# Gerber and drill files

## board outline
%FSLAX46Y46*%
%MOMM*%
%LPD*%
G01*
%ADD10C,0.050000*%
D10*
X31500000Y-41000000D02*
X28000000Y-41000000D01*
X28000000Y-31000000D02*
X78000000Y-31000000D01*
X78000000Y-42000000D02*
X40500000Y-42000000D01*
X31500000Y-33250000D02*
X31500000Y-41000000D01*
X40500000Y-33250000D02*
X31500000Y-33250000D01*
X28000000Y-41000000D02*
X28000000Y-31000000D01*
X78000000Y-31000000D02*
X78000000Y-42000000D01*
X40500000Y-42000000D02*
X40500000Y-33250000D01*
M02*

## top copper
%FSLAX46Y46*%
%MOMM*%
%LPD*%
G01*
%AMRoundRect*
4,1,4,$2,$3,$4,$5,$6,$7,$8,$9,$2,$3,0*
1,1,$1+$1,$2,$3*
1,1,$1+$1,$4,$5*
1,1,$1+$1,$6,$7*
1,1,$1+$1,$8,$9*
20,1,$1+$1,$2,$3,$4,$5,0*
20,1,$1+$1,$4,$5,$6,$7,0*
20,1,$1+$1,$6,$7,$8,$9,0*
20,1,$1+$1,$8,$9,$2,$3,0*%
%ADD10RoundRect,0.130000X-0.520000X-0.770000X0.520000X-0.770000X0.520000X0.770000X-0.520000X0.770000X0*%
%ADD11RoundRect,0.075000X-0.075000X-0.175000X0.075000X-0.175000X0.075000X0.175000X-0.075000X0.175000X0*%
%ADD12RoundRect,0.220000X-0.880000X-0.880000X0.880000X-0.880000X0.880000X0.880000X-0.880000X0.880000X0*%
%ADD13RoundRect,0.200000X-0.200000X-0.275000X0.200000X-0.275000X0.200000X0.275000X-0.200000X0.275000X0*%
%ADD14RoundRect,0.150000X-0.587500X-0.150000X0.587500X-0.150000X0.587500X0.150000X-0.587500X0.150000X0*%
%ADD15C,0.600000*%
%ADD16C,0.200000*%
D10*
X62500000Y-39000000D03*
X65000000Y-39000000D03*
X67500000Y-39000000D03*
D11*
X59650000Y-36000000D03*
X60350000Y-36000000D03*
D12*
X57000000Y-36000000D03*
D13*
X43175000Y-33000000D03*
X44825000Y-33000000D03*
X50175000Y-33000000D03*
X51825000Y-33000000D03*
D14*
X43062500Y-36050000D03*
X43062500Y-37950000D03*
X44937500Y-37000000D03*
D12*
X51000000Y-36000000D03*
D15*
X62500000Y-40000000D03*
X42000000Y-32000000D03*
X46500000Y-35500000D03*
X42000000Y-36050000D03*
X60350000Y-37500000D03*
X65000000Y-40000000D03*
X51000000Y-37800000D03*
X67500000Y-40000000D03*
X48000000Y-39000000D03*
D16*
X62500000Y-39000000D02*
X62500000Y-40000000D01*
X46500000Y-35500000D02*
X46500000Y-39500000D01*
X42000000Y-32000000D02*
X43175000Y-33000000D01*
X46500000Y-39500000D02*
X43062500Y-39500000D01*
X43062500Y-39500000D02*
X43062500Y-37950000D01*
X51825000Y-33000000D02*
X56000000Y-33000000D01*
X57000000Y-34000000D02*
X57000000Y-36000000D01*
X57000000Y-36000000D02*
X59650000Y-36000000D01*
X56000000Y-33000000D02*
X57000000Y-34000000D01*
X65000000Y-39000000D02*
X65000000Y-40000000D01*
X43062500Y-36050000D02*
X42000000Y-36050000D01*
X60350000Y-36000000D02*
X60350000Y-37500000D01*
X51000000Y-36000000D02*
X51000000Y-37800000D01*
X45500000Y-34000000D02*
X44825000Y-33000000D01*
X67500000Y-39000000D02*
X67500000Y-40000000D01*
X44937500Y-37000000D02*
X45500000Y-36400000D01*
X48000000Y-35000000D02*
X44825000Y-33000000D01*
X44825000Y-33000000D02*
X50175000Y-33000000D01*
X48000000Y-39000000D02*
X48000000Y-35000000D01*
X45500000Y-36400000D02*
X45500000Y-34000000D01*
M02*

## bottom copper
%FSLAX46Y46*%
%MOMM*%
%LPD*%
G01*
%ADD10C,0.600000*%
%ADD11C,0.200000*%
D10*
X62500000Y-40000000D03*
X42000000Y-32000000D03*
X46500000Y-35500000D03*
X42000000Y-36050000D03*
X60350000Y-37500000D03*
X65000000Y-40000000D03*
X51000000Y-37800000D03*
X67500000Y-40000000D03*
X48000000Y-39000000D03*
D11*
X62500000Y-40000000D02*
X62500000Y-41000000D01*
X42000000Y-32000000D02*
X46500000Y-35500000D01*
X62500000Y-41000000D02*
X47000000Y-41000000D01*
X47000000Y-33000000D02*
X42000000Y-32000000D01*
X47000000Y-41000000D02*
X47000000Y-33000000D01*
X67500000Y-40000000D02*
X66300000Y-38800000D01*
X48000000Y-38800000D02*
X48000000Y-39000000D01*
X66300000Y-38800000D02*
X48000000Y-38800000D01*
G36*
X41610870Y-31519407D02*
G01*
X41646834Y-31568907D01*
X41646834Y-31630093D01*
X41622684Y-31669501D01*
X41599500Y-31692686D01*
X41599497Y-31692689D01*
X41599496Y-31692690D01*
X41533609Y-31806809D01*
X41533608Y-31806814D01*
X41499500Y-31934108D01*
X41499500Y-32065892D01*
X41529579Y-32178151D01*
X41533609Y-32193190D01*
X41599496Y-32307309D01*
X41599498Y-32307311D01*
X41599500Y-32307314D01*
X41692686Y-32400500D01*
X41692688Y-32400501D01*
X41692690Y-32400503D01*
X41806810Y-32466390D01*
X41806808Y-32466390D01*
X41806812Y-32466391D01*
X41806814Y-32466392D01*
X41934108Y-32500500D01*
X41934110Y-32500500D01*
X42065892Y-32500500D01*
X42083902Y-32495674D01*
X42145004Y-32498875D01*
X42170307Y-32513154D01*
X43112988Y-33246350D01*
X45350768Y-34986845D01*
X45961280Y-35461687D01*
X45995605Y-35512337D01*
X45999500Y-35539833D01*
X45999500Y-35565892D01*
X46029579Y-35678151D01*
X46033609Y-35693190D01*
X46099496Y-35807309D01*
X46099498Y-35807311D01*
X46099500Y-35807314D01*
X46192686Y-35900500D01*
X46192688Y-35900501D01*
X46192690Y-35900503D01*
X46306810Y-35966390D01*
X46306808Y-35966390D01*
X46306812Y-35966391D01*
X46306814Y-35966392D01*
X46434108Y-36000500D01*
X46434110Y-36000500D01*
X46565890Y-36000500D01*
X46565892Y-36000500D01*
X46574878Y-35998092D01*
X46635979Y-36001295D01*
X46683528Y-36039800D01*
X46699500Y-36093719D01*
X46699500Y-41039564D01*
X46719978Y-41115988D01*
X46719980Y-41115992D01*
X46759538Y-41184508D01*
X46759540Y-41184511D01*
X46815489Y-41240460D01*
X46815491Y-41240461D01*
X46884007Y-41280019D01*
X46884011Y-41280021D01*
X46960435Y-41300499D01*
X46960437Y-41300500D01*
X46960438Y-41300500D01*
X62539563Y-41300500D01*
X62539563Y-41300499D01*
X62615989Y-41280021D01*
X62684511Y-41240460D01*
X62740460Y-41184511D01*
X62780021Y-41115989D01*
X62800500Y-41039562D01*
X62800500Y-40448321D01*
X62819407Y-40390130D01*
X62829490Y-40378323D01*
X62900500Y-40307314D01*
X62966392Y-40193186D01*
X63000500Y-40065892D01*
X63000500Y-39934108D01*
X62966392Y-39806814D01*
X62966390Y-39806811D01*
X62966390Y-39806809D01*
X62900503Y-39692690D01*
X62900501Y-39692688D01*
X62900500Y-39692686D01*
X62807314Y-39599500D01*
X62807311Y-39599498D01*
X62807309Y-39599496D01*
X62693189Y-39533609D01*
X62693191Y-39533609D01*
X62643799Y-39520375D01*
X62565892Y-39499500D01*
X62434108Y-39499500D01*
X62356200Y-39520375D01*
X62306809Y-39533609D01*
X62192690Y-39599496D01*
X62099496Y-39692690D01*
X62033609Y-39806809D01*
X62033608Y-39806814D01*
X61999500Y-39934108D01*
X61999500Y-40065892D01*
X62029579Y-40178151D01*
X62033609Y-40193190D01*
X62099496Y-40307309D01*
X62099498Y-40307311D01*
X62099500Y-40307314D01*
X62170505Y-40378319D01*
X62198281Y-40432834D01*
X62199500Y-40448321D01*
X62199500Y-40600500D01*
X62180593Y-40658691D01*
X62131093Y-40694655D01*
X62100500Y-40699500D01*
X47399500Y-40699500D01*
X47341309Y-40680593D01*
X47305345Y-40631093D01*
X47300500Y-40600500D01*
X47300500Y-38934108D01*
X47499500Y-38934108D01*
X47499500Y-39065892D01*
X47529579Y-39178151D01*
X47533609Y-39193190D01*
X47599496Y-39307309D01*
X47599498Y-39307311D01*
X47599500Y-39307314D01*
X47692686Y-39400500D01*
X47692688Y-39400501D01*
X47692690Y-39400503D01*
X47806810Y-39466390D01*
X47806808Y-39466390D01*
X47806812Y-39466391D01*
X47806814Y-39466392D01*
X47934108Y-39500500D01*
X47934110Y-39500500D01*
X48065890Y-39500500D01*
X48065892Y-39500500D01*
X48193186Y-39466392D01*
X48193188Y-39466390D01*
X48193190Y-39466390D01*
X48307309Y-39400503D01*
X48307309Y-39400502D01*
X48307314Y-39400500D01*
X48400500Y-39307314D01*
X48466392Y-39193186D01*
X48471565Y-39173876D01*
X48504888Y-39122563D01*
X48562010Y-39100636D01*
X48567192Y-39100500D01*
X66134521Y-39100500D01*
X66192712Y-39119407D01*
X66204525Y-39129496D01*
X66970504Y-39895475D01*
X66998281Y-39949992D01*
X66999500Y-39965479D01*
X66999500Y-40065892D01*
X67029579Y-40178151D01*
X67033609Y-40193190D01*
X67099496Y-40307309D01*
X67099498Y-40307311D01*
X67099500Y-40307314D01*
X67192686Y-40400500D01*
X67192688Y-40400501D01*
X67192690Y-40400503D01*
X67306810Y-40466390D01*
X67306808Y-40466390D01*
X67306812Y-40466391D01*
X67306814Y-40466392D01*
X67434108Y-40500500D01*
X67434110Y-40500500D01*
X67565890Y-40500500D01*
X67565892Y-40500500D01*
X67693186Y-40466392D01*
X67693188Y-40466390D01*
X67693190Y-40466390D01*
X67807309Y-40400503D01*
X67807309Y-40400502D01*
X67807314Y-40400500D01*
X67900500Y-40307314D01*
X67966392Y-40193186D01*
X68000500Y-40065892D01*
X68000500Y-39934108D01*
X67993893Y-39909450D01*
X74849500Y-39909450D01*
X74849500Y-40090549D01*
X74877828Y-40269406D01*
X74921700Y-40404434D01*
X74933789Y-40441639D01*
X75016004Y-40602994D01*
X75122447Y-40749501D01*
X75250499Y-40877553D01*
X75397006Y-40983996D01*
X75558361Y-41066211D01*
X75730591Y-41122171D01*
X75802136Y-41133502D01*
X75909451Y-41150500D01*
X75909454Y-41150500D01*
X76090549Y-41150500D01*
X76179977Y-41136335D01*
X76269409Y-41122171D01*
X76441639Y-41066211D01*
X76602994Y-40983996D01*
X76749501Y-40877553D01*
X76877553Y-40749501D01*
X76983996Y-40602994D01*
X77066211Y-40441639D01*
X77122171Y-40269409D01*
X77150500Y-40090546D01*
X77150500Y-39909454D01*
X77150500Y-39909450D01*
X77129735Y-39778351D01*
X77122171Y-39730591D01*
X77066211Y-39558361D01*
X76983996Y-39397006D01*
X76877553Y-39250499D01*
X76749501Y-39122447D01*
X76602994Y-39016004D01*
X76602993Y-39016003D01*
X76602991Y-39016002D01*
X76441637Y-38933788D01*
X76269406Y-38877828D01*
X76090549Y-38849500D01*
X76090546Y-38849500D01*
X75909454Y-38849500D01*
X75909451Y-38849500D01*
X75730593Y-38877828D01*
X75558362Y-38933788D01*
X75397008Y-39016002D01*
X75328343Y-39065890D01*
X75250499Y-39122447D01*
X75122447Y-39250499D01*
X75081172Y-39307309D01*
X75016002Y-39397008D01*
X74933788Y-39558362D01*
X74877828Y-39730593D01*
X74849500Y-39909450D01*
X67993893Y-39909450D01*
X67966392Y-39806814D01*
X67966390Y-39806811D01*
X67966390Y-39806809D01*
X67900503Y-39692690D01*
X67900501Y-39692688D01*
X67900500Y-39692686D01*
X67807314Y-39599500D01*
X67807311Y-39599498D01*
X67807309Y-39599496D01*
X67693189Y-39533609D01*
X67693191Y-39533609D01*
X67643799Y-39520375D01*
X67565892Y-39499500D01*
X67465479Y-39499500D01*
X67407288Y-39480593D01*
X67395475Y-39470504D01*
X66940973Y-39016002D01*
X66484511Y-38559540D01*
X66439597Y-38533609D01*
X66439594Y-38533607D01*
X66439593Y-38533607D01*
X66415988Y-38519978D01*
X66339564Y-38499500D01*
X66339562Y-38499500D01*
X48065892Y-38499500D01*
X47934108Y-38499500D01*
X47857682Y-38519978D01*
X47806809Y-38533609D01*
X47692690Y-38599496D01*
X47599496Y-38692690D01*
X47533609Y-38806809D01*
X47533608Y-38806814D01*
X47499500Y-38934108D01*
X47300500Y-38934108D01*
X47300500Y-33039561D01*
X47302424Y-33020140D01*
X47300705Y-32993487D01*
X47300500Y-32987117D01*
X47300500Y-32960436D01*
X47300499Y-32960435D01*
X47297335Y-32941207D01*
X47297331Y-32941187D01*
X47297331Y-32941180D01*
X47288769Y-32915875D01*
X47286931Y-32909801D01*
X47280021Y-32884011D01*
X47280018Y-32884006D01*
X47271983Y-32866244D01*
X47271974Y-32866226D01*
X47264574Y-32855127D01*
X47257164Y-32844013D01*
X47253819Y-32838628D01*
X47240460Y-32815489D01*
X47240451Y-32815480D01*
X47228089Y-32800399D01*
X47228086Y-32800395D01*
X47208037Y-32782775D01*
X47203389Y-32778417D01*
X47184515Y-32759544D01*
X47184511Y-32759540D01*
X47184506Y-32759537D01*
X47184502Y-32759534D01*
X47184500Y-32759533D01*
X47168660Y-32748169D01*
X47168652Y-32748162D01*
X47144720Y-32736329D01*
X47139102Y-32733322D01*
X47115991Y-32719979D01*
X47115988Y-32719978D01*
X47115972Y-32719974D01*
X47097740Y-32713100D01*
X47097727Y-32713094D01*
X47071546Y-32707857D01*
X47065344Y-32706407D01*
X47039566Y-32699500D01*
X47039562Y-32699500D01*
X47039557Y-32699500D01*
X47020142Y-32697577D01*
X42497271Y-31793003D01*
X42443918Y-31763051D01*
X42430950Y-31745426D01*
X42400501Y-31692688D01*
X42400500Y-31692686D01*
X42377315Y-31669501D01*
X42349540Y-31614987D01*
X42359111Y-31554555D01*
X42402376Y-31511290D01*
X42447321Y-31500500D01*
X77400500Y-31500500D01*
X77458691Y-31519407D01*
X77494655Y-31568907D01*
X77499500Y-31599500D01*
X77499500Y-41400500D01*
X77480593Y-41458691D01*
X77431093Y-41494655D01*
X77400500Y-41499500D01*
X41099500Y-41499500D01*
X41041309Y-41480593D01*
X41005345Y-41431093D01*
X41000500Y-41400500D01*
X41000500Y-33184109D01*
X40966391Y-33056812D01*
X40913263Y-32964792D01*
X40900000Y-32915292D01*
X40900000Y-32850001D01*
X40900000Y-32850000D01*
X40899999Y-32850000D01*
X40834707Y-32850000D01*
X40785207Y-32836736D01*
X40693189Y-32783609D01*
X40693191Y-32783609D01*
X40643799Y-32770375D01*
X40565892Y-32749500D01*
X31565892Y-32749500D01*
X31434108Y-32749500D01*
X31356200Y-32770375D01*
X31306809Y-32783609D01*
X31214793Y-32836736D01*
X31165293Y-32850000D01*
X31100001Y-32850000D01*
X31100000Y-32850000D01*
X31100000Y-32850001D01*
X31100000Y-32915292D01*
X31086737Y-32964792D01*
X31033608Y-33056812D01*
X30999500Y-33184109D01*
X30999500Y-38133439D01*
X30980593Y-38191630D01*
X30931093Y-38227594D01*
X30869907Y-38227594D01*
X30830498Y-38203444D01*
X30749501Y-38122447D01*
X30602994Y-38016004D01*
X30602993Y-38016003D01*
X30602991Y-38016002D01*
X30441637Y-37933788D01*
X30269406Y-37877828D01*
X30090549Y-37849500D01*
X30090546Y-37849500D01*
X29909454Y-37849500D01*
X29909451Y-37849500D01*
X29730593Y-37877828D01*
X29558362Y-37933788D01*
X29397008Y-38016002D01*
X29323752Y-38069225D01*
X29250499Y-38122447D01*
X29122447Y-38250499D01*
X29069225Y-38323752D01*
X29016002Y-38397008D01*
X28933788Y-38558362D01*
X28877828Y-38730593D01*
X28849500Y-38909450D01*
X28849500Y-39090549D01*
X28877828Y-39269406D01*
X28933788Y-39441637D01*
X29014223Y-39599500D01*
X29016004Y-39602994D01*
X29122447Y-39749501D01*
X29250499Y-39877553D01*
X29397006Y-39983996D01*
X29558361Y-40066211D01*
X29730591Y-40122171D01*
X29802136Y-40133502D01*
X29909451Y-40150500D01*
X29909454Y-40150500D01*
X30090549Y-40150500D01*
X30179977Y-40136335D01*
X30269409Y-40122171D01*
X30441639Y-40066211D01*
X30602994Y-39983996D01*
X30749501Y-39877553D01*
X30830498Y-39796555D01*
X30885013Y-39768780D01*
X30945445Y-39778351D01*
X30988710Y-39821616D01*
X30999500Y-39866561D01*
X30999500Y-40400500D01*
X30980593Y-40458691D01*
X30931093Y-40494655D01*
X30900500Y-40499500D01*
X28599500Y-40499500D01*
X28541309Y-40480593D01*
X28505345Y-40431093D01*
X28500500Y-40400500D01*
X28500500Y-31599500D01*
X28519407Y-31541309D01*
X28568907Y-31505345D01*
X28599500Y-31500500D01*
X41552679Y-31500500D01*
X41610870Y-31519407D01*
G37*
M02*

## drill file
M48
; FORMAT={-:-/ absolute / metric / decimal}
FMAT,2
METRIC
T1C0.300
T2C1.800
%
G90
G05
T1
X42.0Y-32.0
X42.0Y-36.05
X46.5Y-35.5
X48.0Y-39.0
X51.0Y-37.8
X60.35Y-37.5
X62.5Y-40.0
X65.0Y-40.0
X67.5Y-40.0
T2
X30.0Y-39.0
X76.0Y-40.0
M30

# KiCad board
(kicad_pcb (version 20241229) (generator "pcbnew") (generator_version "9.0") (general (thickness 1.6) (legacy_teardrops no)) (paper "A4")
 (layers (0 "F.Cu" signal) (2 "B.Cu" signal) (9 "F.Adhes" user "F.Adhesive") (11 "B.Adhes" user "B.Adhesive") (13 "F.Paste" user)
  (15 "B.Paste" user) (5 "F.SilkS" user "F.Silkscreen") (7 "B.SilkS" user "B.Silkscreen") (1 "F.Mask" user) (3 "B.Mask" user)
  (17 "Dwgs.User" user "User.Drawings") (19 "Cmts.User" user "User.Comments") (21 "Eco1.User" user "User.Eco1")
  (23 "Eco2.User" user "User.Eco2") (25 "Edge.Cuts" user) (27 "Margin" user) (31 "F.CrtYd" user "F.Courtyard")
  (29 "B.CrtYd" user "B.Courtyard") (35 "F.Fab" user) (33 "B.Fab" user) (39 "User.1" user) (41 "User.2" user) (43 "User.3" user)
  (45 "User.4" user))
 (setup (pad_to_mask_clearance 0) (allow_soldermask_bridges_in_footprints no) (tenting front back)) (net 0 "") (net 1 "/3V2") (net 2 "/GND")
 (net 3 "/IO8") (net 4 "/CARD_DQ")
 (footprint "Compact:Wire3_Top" (layer "F.Cu") (at 65 39)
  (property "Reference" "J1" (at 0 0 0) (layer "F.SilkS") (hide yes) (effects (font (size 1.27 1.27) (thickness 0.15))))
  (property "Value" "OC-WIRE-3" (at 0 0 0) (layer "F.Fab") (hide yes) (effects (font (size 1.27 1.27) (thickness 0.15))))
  (pad "1" smd roundrect (at -2.5 0) (size 1.3 1.8) (layers "F.Cu" "F.Mask") (roundrect_rratio 0.1) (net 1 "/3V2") (thermal_bridge_angle 45))
  (pad "2" smd roundrect (at 0 0) (size 1.3 1.8) (layers "F.Cu" "F.Mask") (roundrect_rratio 0.1) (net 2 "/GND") (thermal_bridge_angle 45))
  (pad "3" smd roundrect (at 2.5 0) (size 1.3 1.8) (layers "F.Cu" "F.Mask") (roundrect_rratio 0.1) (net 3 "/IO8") (thermal_bridge_angle 45)))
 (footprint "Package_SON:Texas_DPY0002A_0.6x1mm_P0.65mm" (layer "F.Cu") (at 60 36)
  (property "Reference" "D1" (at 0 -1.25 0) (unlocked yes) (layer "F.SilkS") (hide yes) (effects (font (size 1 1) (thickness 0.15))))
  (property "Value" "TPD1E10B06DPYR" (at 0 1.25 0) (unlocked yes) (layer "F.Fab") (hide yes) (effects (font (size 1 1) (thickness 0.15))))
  (pad "1" smd roundrect (at -0.35 0) (size 0.3 0.5) (layers "F.Cu" "F.Mask" "F.Paste") (roundrect_rratio 0.25) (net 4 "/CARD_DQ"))
  (pad "2" smd roundrect (at 0.35 0) (size 0.3 0.5) (layers "F.Cu" "F.Mask" "F.Paste") (roundrect_rratio 0.25) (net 2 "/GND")))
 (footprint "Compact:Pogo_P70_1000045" (layer "F.Cu") (at 57 36)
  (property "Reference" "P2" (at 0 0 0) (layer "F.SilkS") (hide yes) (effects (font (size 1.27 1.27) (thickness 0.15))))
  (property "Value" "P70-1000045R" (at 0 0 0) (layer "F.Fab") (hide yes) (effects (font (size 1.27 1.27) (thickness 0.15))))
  (pad "1" smd roundrect (at 0 0) (size 2.2 2.2) (layers "F.Cu" "F.Mask" "F.Paste") (roundrect_rratio 0.1) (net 4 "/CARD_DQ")
   (thermal_bridge_angle 45)))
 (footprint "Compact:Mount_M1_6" (layer "F.Cu") (at 30 39)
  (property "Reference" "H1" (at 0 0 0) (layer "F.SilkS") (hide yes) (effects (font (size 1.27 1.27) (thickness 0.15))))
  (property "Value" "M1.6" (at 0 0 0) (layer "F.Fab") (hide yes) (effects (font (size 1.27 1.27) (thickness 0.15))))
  (pad "" np_thru_hole circle (at 0 0) (size 1.8 1.8) (drill 1.8) (layers "*.Cu")))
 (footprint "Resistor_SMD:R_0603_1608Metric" (layer "F.Cu") (at 44 33)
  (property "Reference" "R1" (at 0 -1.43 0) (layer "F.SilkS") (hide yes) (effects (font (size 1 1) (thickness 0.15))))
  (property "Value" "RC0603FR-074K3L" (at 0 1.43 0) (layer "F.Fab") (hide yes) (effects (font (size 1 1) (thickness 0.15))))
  (pad "1" smd roundrect (at -0.825 0) (size 0.8 0.95) (layers "F.Cu" "F.Mask" "F.Paste") (roundrect_rratio 0.25) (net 1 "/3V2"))
  (pad "2" smd roundrect (at 0.825 0) (size 0.8 0.95) (layers "F.Cu" "F.Mask" "F.Paste") (roundrect_rratio 0.25) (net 3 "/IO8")))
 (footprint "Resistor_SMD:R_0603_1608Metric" (layer "F.Cu") (at 51 33)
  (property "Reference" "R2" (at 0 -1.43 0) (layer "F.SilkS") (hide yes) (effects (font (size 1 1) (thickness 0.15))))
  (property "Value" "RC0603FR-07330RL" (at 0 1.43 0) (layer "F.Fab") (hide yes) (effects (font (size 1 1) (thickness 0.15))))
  (pad "1" smd roundrect (at -0.825 0) (size 0.8 0.95) (layers "F.Cu" "F.Mask" "F.Paste") (roundrect_rratio 0.25) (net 3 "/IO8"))
  (pad "2" smd roundrect (at 0.825 0) (size 0.8 0.95) (layers "F.Cu" "F.Mask" "F.Paste") (roundrect_rratio 0.25) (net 4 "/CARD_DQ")))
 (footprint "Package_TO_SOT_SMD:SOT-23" (layer "F.Cu") (at 44 37)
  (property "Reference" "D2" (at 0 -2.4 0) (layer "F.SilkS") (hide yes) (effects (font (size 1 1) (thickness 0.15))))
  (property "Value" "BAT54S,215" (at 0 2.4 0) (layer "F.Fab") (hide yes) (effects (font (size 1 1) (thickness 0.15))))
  (pad "1" smd roundrect (at -0.9375 -0.95) (size 1.475 0.6) (layers "F.Cu" "F.Mask" "F.Paste") (roundrect_rratio 0.25) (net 2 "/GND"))
  (pad "2" smd roundrect (at -0.9375 0.95) (size 1.475 0.6) (layers "F.Cu" "F.Mask" "F.Paste") (roundrect_rratio 0.25) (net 1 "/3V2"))
  (pad "3" smd roundrect (at 0.9375 0) (size 1.475 0.6) (layers "F.Cu" "F.Mask" "F.Paste") (roundrect_rratio 0.25) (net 3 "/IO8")))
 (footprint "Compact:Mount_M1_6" (layer "F.Cu") (at 76 40)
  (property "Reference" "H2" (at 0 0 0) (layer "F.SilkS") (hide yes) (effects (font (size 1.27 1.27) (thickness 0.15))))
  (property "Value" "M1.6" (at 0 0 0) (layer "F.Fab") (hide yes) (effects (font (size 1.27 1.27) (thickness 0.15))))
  (pad "" np_thru_hole circle (at 0 0) (size 1.8 1.8) (drill 1.8) (layers "*.Cu")))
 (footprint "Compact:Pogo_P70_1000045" (layer "F.Cu") (at 51 36)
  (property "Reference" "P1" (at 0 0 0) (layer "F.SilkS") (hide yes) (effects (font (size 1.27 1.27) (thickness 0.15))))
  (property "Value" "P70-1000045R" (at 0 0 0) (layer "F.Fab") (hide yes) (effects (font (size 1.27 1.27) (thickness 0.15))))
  (pad "1" smd roundrect (at 0 0) (size 2.2 2.2) (layers "F.Cu" "F.Mask" "F.Paste") (roundrect_rratio 0.1) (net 2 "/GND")
   (thermal_bridge_angle 45)))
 (gr_line (start 31.5 41) (end 28 41) (stroke (width 0.05) (type default)) (layer "Edge.Cuts"))
 (gr_line (start 28 31) (end 78 31) (stroke (width 0.05) (type default)) (layer "Edge.Cuts"))
 (gr_line (start 78 42) (end 40.5 42) (stroke (width 0.05) (type default)) (layer "Edge.Cuts"))
 (gr_line (start 31.5 33.25) (end 31.5 41) (stroke (width 0.05) (type default)) (layer "Edge.Cuts"))
 (gr_line (start 40.5 33.25) (end 31.5 33.25) (stroke (width 0.05) (type default)) (layer "Edge.Cuts"))
 (gr_line (start 28 41) (end 28 31) (stroke (width 0.05) (type default)) (layer "Edge.Cuts"))
 (gr_line (start 78 31) (end 78 42) (stroke (width 0.05) (type default)) (layer "Edge.Cuts"))
 (gr_line (start 40.5 42) (end 40.5 33.25) (stroke (width 0.05) (type default)) (layer "Edge.Cuts"))
 (segment (start 62.5 39) (end 62.5 40) (width 0.2) (layer "F.Cu") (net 1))
 (segment (start 46.5 35.5) (end 46.5 39.5) (width 0.2) (layer "F.Cu") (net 1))
 (segment (start 42 32) (end 43.175 33) (width 0.2) (layer "F.Cu") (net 1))
 (segment (start 46.5 39.5) (end 43.0625 39.5) (width 0.2) (layer "F.Cu") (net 1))
 (segment (start 43.0625 39.5) (end 43.0625 37.95) (width 0.2) (layer "F.Cu") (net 1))
 (via (at 62.5 40) (size 0.6) (drill 0.3) (layers "F.Cu" "B.Cu") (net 1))
 (via (at 42 32) (size 0.6) (drill 0.3) (layers "F.Cu" "B.Cu") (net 1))
 (via (at 46.5 35.5) (size 0.6) (drill 0.3) (layers "F.Cu" "B.Cu") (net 1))
 (segment (start 62.5 40) (end 62.5 41) (width 0.2) (layer "B.Cu") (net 1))
 (segment (start 42 32) (end 46.5 35.5) (width 0.2) (layer "B.Cu") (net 1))
 (segment (start 62.5 41) (end 47 41) (width 0.2) (layer "B.Cu") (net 1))
 (segment (start 47 33) (end 42 32) (width 0.2) (layer "B.Cu") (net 1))
 (segment (start 47 41) (end 47 33) (width 0.2) (layer "B.Cu") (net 1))
 (segment (start 51.825 33) (end 56 33) (width 0.2) (layer "F.Cu") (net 4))
 (segment (start 57 34) (end 57 36) (width 0.2) (layer "F.Cu") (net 4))
 (segment (start 57 36) (end 59.65 36) (width 0.2) (layer "F.Cu") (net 4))
 (segment (start 56 33) (end 57 34) (width 0.2) (layer "F.Cu") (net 4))
 (segment (start 65 39) (end 65 40) (width 0.2) (layer "F.Cu") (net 2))
 (segment (start 43.0625 36.05) (end 42 36.05) (width 0.2) (layer "F.Cu") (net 2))
 (segment (start 60.35 36) (end 60.35 37.5) (width 0.2) (layer "F.Cu") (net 2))
 (segment (start 51 36) (end 51 37.8) (width 0.2) (layer "F.Cu") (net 2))
 (via (at 42 36.05) (size 0.6) (drill 0.3) (layers "F.Cu" "B.Cu") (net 2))
 (via (at 60.35 37.5) (size 0.6) (drill 0.3) (layers "F.Cu" "B.Cu") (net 2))
 (via (at 65 40) (size 0.6) (drill 0.3) (layers "F.Cu" "B.Cu") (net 2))
 (via (at 51 37.8) (size 0.6) (drill 0.3) (layers "F.Cu" "B.Cu") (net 2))
 (segment (start 45.5 34) (end 44.825 33) (width 0.2) (layer "F.Cu") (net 3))
 (segment (start 67.5 39) (end 67.5 40) (width 0.2) (layer "F.Cu") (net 3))
 (segment (start 44.9375 37) (end 45.5 36.4) (width 0.2) (layer "F.Cu") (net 3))
 (segment (start 48 35) (end 44.825 33) (width 0.2) (layer "F.Cu") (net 3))
 (segment (start 44.825 33) (end 50.175 33) (width 0.2) (layer "F.Cu") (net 3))
 (segment (start 48 39) (end 48 35) (width 0.2) (layer "F.Cu") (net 3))
 (segment (start 45.5 36.4) (end 45.5 34) (width 0.2) (layer "F.Cu") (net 3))
 (via (at 67.5 40) (size 0.6) (drill 0.3) (layers "F.Cu" "B.Cu") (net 3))
 (via (at 48 39) (size 0.6) (drill 0.3) (layers "F.Cu" "B.Cu") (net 3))
 (segment (start 67.5 40) (end 66.3 38.8) (width 0.2) (layer "B.Cu") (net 3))
 (segment (start 48 38.8) (end 48 39) (width 0.2) (layer "B.Cu") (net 3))
 (segment (start 66.3 38.8) (end 48 38.8) (width 0.2) (layer "B.Cu") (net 3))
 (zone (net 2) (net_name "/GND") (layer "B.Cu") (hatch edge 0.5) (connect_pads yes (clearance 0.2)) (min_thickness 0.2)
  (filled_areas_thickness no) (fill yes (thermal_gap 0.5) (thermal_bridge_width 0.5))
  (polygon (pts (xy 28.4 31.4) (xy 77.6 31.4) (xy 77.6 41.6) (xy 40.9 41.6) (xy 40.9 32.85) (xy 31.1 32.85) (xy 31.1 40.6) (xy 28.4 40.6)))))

